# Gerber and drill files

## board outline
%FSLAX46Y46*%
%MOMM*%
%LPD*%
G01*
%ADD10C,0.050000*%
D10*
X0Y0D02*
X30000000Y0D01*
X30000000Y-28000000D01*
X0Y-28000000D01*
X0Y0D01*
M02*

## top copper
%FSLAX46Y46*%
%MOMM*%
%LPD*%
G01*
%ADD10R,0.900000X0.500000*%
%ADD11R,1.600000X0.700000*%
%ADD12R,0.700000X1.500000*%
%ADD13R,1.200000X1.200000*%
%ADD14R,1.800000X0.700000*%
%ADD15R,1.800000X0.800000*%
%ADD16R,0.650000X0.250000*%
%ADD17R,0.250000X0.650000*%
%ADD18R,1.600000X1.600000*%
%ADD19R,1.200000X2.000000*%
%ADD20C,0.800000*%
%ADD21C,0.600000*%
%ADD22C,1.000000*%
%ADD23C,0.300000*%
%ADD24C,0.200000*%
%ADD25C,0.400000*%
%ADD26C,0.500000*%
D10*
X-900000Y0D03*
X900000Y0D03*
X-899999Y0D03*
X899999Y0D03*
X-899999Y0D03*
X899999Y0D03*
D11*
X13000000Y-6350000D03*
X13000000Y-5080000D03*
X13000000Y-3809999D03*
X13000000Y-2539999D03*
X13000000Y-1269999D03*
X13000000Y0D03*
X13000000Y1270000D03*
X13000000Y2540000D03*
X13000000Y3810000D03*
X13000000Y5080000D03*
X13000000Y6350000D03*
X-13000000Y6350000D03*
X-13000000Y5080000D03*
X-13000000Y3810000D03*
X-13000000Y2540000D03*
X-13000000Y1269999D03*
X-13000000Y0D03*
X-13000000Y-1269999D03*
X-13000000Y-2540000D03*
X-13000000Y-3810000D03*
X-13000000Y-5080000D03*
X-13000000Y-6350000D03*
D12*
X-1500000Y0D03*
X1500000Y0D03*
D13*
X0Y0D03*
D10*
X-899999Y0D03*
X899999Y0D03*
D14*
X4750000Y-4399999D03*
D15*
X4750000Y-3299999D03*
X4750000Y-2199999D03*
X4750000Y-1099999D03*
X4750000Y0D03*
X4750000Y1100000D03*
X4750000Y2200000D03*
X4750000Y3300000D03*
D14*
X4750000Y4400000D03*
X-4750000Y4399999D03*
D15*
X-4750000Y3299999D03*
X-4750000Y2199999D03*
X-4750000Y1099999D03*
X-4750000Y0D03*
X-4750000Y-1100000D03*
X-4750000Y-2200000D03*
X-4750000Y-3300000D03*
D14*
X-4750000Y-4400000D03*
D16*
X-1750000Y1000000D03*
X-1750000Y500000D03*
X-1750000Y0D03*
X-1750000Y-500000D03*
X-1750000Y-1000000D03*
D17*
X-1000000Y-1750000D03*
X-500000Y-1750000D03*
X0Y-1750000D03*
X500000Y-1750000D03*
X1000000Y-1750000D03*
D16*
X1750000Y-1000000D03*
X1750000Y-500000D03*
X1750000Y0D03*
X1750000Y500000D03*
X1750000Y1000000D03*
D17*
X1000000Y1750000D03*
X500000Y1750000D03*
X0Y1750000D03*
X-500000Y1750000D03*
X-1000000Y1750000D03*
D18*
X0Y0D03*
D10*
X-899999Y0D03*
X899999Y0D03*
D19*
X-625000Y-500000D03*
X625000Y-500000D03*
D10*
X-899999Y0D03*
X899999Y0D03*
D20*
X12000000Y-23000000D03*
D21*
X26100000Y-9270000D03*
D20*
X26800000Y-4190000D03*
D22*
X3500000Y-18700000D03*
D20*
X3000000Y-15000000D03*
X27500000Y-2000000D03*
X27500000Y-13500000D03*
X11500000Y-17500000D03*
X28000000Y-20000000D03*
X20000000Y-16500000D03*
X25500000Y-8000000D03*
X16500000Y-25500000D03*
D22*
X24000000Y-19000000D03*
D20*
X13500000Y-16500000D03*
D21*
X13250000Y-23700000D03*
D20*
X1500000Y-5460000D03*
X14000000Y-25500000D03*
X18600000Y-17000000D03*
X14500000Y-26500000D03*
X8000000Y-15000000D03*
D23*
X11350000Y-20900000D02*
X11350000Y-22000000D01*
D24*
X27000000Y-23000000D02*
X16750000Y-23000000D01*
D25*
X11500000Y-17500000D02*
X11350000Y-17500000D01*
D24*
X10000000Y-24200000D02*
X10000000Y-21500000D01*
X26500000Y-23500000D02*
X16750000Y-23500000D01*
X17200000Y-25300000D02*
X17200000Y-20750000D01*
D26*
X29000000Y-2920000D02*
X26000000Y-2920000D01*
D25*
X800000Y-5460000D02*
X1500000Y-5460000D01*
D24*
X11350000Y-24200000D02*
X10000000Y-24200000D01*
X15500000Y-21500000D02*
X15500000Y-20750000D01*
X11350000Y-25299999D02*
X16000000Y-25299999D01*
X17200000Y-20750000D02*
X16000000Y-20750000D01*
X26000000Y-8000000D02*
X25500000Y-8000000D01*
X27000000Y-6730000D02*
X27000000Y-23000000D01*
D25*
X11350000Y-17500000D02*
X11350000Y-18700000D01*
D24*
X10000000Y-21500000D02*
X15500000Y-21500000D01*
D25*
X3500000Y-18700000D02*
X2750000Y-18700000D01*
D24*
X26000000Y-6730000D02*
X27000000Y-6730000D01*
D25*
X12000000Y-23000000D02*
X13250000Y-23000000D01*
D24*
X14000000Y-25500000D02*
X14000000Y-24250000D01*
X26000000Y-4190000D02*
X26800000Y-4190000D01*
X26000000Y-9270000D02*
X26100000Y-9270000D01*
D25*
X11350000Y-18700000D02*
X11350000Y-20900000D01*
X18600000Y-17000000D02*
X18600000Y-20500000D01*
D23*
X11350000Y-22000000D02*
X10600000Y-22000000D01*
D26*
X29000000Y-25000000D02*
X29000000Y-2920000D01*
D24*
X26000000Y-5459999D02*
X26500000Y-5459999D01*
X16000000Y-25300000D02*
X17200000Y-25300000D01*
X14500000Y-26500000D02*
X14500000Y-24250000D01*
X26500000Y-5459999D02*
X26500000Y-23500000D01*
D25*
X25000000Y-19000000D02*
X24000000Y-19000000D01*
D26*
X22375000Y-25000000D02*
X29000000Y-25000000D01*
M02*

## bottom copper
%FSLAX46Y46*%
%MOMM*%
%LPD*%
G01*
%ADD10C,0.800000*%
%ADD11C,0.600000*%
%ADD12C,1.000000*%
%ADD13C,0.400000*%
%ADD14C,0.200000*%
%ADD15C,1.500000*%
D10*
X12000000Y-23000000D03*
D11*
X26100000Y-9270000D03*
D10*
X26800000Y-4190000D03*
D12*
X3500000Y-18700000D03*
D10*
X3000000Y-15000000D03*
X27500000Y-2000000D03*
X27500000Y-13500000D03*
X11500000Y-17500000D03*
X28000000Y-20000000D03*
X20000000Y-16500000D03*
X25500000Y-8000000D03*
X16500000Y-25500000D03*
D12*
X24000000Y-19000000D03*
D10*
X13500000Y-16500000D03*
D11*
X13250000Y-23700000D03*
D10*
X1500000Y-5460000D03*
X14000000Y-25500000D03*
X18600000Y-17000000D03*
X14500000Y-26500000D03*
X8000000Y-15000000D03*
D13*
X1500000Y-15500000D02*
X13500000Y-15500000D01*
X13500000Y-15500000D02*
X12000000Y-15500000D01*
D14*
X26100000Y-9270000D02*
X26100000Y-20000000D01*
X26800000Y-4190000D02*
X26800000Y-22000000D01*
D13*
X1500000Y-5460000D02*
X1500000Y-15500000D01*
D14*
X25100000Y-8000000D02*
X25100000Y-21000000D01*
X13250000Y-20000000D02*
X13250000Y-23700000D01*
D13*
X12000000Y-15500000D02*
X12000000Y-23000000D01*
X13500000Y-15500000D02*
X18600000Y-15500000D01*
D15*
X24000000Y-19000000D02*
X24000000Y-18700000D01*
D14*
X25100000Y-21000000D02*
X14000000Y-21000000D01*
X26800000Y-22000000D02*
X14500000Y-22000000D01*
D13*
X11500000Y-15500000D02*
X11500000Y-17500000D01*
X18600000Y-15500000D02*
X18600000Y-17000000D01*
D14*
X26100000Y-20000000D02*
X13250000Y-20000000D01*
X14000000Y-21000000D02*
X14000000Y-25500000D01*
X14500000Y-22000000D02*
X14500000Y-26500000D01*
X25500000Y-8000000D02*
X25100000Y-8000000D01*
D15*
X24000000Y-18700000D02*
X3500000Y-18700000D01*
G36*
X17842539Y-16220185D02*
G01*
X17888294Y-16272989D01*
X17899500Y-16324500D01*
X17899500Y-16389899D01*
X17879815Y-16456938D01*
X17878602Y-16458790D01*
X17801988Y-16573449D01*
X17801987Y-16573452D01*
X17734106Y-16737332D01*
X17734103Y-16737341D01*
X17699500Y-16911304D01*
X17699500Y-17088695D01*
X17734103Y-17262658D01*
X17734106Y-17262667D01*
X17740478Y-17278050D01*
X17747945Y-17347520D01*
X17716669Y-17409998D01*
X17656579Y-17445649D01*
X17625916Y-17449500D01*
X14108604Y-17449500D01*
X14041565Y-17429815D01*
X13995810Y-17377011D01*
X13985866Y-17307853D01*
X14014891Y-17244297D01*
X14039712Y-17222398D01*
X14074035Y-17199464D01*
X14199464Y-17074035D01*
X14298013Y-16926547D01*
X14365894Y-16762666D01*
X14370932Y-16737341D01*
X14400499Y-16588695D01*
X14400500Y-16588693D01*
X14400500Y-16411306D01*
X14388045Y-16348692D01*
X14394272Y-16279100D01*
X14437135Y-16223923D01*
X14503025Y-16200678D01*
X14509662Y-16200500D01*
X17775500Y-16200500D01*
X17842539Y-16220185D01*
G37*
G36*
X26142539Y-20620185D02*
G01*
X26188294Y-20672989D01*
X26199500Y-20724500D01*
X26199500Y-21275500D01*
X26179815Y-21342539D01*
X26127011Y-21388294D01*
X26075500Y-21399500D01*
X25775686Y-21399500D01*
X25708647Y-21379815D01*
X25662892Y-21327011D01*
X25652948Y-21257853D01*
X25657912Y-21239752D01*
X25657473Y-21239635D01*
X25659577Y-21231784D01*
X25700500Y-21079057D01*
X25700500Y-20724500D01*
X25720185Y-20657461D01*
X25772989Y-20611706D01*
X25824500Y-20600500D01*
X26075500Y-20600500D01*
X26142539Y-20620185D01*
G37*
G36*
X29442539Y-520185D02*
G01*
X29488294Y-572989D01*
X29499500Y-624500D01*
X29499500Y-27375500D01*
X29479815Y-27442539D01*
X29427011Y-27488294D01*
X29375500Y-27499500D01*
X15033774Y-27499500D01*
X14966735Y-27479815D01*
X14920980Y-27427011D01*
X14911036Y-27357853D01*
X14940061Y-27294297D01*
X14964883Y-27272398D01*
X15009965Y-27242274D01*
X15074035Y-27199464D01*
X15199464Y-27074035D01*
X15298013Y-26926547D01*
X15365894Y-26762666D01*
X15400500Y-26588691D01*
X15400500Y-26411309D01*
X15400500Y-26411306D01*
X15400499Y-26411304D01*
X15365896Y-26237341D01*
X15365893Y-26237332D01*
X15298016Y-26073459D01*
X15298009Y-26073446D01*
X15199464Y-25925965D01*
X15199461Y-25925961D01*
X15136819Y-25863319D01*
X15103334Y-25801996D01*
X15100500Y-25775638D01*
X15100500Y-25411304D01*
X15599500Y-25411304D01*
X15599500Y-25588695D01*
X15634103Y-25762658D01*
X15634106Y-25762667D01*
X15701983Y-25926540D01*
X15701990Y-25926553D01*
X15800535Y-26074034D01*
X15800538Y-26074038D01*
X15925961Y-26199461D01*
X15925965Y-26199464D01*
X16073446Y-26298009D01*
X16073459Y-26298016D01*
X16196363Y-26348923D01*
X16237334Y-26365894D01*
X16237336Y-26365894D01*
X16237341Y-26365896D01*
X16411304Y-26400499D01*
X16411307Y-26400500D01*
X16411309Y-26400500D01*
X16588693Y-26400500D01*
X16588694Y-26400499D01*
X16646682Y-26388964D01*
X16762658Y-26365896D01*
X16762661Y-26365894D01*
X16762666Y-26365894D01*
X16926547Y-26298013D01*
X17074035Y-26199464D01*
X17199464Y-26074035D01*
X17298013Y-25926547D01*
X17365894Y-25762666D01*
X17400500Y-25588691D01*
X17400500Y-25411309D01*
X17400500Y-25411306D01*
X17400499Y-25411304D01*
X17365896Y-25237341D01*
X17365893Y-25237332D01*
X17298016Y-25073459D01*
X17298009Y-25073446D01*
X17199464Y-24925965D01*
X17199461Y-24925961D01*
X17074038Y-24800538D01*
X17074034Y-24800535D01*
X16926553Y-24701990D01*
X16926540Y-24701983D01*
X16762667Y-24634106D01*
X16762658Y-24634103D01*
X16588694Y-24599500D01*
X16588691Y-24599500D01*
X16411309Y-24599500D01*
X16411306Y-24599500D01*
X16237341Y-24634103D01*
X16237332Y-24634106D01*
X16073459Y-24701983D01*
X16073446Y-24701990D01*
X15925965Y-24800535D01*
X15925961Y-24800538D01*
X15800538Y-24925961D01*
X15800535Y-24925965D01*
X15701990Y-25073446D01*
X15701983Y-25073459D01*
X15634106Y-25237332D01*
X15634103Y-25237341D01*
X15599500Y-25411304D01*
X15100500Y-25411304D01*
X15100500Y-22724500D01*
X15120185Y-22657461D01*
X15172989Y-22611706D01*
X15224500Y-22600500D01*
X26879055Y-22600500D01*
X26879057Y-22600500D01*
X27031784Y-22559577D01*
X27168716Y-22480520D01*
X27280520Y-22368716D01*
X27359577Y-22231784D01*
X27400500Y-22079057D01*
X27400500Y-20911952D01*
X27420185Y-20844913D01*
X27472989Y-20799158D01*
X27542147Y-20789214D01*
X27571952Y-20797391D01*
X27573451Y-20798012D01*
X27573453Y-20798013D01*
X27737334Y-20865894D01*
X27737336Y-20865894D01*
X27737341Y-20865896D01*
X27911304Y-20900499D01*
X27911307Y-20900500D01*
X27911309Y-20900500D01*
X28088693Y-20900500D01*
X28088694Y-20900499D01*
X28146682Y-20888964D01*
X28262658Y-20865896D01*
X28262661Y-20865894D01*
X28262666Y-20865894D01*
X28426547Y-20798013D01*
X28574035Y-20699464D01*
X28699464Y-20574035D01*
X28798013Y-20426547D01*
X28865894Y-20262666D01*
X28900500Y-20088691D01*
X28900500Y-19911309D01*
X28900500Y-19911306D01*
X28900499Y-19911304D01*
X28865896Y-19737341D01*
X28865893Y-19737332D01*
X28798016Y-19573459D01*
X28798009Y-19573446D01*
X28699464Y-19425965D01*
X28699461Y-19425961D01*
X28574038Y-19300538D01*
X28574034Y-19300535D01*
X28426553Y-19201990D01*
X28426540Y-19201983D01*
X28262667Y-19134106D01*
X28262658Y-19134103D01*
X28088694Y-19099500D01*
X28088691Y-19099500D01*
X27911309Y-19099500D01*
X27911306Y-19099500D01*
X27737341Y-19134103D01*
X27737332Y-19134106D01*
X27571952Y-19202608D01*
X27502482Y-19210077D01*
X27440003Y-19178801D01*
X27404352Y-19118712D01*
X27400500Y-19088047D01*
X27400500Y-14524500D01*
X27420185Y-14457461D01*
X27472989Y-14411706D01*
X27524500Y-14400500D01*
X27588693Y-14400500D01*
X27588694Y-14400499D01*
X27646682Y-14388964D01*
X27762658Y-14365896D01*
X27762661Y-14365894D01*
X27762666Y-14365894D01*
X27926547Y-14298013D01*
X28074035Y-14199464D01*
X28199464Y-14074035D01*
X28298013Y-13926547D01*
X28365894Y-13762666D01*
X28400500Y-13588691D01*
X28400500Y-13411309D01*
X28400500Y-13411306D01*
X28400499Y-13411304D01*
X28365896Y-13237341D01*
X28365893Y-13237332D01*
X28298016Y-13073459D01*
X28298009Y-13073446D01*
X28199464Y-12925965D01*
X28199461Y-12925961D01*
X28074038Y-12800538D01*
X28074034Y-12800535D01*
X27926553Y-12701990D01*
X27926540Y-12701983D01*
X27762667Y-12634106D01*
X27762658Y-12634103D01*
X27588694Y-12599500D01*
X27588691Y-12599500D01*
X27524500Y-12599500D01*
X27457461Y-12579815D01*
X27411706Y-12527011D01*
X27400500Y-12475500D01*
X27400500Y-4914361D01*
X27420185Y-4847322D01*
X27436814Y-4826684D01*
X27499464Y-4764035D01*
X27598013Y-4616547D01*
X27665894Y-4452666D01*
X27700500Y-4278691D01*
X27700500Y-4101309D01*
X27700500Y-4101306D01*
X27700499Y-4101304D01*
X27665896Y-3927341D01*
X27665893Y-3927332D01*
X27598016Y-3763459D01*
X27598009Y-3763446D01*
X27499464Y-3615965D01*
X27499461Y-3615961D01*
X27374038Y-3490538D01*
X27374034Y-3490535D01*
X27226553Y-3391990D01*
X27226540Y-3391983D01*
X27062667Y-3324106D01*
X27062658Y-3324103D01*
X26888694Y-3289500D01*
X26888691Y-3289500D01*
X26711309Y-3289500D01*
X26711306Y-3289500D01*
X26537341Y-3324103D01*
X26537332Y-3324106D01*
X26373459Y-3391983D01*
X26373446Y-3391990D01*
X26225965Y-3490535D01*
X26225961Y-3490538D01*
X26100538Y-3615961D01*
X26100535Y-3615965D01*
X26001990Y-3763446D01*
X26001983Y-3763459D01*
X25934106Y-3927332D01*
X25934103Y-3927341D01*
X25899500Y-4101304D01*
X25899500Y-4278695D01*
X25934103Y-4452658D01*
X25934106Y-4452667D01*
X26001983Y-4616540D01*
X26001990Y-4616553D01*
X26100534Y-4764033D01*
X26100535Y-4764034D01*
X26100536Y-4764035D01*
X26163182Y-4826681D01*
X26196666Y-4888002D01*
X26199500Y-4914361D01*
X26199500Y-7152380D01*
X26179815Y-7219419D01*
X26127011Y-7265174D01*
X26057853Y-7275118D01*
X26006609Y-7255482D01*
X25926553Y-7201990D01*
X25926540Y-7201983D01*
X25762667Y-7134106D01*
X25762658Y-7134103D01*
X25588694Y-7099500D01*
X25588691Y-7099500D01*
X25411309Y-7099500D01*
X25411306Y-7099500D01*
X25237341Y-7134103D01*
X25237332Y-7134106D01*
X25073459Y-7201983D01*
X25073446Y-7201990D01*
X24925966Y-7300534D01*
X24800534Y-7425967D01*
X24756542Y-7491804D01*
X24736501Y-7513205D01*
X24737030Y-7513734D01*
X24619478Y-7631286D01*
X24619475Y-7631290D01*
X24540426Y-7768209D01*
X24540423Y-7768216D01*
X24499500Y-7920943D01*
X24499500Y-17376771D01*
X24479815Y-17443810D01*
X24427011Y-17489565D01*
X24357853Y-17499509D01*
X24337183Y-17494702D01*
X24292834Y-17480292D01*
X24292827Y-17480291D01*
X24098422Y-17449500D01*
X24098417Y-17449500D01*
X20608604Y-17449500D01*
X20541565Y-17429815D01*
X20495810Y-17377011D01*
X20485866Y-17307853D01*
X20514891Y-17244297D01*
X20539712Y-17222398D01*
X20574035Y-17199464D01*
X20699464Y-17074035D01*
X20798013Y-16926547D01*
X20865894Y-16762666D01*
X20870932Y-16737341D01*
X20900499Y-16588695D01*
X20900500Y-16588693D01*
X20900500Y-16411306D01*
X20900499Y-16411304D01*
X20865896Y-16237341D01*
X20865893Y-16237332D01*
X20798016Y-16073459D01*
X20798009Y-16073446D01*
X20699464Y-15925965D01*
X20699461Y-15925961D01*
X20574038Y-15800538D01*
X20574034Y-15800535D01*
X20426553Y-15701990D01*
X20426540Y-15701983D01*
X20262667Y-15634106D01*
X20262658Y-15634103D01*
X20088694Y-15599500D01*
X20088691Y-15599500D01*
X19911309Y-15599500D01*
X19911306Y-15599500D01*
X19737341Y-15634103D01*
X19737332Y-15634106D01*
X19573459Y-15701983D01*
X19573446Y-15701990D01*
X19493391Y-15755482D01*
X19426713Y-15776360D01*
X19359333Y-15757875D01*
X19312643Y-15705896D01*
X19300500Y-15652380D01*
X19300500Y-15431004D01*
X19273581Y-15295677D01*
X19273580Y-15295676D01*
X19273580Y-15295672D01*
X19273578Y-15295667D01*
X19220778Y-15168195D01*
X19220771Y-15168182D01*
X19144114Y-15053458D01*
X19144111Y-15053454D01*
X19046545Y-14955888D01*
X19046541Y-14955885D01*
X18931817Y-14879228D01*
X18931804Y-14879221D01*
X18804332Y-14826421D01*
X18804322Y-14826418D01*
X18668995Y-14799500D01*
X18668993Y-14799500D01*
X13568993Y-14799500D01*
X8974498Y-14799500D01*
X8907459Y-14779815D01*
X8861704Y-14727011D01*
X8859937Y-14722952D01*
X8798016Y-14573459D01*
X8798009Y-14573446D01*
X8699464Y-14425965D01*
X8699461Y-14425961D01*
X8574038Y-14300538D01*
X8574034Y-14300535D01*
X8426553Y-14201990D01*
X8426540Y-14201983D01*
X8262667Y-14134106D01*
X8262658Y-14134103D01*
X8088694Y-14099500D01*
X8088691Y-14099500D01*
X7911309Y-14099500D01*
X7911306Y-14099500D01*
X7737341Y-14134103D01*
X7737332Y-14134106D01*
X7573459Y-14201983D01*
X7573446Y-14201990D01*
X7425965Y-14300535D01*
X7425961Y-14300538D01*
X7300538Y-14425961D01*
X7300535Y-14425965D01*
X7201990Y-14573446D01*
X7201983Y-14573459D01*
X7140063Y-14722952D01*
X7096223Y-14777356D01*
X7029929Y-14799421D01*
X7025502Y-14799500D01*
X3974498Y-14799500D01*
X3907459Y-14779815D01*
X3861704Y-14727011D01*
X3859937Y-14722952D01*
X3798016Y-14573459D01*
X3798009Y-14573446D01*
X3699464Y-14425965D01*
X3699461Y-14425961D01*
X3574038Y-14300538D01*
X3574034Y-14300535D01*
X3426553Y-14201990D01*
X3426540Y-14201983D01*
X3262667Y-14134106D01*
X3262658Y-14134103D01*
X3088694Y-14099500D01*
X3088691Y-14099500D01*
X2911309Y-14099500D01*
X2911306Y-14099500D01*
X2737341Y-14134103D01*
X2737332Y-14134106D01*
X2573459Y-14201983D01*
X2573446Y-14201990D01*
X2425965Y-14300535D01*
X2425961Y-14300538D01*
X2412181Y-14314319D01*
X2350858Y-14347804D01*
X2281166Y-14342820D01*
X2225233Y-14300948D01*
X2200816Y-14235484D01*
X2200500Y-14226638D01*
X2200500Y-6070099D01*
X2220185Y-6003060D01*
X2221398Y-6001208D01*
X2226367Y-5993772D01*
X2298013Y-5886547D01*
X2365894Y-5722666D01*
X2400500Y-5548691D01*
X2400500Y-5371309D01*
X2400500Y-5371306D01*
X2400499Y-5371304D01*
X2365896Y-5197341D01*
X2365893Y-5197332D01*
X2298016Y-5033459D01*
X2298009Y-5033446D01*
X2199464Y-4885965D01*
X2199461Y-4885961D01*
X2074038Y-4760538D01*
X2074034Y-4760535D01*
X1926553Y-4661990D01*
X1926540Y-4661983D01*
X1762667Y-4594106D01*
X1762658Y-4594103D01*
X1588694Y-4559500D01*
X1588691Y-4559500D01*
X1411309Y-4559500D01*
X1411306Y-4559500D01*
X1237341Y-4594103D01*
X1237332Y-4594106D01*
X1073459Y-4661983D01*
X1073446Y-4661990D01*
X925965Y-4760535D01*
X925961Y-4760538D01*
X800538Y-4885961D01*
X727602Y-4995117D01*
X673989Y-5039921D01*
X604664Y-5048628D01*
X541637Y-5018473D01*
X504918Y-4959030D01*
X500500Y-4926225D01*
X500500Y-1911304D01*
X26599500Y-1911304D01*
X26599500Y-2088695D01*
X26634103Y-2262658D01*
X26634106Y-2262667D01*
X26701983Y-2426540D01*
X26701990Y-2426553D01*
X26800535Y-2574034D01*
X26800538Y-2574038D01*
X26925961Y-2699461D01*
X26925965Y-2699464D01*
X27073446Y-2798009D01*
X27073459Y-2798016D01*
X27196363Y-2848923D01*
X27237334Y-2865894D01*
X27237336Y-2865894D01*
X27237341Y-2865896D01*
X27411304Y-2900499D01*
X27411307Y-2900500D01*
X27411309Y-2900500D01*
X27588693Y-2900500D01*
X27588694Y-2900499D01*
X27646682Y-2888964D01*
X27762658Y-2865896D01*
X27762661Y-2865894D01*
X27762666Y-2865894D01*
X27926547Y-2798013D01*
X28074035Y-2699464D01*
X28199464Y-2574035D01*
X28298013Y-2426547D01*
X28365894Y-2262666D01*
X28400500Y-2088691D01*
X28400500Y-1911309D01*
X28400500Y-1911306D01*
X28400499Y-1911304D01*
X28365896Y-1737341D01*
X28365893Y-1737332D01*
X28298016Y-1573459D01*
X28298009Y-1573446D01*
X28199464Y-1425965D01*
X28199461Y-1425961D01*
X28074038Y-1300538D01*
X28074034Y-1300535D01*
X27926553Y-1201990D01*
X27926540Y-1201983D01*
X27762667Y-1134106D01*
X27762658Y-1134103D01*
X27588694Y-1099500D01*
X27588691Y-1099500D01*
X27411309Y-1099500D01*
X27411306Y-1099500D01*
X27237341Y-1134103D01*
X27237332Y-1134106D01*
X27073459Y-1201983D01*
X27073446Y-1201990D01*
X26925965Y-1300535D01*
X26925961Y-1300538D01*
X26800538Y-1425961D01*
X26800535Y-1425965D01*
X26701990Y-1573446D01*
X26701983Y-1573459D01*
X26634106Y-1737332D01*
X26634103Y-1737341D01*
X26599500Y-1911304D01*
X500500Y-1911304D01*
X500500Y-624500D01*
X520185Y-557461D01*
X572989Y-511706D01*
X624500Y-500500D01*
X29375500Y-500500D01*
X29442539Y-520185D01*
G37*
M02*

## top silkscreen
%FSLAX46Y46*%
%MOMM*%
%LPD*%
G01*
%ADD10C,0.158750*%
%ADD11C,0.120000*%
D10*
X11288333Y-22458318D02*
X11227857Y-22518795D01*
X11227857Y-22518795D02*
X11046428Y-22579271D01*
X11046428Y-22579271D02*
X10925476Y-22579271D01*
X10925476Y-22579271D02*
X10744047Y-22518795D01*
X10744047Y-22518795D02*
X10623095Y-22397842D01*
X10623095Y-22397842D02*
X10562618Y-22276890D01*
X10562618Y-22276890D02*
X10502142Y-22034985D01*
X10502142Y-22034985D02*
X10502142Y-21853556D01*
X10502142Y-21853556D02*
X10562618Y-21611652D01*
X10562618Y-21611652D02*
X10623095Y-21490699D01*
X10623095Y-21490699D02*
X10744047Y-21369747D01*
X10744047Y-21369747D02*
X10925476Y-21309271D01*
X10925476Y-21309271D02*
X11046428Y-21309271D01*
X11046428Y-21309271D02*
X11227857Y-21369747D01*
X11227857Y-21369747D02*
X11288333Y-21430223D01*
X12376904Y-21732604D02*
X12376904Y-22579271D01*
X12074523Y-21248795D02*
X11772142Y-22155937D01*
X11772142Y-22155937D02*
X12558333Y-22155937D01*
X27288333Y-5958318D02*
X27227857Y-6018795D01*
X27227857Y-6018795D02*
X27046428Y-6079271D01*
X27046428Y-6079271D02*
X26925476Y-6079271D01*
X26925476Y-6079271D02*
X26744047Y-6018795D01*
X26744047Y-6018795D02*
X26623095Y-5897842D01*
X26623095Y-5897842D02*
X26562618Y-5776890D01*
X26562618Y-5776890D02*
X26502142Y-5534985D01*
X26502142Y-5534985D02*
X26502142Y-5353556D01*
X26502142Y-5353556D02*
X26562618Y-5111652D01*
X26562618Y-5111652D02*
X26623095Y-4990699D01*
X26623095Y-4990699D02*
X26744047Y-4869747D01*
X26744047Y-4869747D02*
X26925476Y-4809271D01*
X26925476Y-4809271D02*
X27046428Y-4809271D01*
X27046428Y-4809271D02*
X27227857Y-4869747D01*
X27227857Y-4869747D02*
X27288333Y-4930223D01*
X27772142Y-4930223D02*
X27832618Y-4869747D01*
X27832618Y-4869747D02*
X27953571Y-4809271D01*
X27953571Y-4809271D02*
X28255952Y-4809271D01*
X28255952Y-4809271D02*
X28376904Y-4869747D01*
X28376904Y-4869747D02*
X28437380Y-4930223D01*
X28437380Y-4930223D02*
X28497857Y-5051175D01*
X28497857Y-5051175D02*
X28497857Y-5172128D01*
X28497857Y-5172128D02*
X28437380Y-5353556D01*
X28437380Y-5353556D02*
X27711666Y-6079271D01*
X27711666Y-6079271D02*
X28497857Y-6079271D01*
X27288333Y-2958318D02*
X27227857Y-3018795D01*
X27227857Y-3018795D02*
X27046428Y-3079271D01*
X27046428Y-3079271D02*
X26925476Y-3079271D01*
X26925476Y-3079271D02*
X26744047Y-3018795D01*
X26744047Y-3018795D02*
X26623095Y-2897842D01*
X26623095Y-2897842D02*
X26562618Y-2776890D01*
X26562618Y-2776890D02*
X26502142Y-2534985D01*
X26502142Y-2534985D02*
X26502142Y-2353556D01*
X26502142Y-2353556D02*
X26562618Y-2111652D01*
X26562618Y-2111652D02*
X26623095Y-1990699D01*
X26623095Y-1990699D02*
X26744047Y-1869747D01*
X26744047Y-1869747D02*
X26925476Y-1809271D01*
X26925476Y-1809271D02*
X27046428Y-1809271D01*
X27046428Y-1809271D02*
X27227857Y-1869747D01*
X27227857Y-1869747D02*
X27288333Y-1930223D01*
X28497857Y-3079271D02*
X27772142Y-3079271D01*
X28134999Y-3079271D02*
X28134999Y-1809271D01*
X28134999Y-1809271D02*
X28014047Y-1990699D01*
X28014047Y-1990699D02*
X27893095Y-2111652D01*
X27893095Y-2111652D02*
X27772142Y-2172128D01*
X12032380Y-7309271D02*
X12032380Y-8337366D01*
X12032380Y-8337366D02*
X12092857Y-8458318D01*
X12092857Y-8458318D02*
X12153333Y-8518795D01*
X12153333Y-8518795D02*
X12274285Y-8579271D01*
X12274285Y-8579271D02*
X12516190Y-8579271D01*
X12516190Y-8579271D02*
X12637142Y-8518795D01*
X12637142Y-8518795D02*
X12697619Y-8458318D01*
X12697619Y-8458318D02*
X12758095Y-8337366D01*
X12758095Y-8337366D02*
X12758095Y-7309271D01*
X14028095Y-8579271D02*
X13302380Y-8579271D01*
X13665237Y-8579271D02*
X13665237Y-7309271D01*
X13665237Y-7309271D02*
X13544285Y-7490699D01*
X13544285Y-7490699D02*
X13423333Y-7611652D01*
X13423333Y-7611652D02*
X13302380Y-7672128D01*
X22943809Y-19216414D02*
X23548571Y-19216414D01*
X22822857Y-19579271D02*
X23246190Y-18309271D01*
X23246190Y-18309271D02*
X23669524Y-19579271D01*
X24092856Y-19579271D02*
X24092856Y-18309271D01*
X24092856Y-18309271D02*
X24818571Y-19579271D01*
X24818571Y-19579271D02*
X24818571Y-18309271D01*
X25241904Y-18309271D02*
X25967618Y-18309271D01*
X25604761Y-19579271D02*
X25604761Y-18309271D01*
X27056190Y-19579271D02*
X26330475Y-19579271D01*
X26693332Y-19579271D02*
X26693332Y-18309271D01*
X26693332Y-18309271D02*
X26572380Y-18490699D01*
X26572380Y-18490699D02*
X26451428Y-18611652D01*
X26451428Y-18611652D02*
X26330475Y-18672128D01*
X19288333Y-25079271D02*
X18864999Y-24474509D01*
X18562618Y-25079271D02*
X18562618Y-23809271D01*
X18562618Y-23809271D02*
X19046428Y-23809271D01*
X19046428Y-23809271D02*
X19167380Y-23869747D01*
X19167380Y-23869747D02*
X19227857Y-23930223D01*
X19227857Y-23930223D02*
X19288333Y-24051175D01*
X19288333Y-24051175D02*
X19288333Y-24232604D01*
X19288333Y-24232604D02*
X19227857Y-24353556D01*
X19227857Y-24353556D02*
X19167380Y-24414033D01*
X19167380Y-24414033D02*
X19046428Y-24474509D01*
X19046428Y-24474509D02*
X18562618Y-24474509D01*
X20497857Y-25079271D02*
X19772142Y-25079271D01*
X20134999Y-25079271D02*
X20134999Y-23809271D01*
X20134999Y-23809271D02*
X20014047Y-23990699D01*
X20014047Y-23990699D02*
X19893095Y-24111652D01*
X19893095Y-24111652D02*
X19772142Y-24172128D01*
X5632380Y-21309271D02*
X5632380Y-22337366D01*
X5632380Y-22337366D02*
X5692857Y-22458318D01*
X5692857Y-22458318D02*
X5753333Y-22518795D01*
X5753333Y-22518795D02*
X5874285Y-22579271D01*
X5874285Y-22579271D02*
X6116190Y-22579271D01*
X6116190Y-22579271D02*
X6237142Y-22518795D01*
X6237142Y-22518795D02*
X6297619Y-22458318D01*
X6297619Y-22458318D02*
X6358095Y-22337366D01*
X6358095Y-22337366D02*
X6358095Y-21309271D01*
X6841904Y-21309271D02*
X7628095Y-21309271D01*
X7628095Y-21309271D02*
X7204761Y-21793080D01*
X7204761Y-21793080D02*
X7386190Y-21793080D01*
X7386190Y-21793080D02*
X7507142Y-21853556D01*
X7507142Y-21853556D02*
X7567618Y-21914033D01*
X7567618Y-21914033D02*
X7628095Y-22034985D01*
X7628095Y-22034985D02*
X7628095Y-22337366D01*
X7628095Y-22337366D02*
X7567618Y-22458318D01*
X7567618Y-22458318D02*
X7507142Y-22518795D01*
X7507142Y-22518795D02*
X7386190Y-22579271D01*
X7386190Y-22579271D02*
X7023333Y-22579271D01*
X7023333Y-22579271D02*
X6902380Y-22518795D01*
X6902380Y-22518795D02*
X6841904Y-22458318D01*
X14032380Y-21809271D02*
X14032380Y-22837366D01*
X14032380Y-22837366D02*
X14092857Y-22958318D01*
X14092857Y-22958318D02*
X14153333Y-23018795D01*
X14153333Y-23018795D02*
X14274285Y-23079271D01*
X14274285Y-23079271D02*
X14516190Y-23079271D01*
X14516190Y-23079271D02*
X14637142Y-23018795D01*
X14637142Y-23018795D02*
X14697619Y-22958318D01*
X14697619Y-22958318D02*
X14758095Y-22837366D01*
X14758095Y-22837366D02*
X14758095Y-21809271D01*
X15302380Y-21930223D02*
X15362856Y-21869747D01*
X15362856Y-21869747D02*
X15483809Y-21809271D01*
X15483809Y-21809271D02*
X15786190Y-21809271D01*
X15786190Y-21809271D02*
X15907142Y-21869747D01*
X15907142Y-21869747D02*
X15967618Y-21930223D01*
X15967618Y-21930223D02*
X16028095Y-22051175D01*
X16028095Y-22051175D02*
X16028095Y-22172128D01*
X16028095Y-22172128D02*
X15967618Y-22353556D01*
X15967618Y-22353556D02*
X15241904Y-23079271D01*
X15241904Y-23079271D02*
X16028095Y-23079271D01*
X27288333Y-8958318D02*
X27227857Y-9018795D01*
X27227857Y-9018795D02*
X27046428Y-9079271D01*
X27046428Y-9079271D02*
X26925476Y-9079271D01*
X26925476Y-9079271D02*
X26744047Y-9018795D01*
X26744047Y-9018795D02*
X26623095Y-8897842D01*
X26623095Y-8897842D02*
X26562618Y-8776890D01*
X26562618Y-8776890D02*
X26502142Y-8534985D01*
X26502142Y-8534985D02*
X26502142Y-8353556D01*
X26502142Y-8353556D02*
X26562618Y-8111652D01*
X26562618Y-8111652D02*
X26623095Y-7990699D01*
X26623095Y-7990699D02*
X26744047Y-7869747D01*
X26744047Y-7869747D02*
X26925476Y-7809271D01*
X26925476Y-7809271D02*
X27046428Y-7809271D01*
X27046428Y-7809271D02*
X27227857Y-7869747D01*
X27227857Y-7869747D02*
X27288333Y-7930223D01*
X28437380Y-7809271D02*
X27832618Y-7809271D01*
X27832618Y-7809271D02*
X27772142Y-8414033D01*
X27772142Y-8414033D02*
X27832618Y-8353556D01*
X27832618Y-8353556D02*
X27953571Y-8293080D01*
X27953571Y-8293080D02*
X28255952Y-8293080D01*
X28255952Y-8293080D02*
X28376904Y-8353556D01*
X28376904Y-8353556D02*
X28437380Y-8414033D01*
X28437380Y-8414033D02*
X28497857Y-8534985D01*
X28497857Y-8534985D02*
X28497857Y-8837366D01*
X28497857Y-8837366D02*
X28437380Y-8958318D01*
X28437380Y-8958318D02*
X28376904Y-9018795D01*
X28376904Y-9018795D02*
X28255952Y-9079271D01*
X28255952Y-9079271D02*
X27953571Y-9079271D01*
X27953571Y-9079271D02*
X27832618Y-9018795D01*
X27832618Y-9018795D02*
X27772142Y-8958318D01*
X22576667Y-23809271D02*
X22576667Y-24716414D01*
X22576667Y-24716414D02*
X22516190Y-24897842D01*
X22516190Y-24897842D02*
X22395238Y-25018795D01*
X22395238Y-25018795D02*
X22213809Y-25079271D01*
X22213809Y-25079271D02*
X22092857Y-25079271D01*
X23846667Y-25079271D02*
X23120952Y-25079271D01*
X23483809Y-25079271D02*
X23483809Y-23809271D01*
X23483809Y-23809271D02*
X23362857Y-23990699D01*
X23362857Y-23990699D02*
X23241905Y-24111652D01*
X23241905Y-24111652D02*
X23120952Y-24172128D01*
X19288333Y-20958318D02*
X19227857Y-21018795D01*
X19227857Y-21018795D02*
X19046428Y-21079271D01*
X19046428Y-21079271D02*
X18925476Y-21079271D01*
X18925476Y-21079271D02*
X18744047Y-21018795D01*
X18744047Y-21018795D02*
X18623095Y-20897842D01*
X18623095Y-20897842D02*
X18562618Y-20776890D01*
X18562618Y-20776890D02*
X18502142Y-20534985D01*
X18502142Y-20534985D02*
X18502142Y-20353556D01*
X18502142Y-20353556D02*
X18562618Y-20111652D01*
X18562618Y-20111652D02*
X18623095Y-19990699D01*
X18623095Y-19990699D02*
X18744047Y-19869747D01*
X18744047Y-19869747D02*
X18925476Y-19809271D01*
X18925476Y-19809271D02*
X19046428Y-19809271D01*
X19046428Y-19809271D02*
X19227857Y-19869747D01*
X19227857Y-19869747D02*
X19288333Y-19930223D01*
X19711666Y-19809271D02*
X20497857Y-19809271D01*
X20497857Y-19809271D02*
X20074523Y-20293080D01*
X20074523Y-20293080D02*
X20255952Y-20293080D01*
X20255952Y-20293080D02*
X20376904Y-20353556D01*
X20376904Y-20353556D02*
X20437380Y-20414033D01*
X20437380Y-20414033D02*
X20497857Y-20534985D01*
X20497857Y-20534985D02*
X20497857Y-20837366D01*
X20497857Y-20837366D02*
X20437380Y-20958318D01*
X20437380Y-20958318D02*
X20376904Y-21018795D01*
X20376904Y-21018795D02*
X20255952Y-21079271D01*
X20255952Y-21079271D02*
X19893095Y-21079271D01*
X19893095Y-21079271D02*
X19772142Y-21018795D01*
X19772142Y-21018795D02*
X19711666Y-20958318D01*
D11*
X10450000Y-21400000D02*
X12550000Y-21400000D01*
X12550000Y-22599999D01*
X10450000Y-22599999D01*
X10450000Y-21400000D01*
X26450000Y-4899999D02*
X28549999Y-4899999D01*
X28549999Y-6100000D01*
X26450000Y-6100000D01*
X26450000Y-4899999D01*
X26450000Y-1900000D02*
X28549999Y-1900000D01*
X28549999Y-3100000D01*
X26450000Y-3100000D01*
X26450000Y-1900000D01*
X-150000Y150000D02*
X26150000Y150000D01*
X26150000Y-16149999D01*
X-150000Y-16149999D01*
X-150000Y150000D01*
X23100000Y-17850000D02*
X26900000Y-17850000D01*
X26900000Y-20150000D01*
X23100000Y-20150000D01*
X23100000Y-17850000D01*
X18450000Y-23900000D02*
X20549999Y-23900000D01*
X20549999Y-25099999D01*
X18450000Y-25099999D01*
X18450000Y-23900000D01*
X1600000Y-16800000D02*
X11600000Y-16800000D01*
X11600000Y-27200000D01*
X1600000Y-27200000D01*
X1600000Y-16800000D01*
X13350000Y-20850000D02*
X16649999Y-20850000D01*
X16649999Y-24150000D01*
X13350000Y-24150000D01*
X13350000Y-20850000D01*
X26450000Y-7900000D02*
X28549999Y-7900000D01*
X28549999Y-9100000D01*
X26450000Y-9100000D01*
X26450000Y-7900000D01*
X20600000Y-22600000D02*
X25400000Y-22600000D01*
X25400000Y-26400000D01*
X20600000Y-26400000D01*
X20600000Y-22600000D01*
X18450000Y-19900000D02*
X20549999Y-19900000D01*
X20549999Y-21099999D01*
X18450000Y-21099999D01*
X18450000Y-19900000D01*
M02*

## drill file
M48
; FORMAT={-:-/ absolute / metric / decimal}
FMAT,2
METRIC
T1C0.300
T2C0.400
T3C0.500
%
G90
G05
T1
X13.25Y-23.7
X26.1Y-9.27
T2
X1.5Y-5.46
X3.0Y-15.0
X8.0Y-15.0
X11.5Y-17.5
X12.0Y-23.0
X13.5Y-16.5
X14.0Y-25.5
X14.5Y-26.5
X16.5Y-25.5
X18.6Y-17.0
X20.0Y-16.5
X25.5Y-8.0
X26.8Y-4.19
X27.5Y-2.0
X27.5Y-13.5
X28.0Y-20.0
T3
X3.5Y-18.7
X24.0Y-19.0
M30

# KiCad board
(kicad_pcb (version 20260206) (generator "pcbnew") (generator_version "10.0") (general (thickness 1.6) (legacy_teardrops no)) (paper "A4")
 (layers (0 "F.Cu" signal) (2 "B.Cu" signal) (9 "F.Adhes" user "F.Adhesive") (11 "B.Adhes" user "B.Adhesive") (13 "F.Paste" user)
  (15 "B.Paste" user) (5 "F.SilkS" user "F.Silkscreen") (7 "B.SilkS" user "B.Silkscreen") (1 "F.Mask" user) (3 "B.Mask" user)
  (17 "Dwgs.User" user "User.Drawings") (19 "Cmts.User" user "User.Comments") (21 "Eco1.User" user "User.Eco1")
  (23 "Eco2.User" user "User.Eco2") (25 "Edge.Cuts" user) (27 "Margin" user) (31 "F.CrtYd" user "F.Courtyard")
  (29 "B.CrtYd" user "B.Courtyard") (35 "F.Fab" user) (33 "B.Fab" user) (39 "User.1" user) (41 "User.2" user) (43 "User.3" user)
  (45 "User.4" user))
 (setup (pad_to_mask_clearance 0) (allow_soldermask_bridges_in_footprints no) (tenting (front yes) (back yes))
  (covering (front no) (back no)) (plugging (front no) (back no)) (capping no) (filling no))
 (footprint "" (layer "F.Cu") (at 11.5 22)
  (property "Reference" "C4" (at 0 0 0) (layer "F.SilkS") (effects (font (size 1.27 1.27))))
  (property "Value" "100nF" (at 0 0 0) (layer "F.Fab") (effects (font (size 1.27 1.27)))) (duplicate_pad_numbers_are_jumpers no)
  (fp_rect (start -1.05 -0.6) (end 1.05 0.599999) (stroke (width 0.12) (type default)) (fill no) (layer "F.SilkS"))
  (pad "1" smd rect (at -12.4 -22) (size 0.9 0.5) (layers "F.Cu" "F.Mask" "F.Paste") (thermal_bridge_angle 45))
  (pad "2" smd rect (at -10.6 -22) (size 0.9 0.5) (layers "F.Cu" "F.Mask" "F.Paste") (thermal_bridge_angle 45)))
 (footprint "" (layer "F.Cu") (at 27.5 5.5)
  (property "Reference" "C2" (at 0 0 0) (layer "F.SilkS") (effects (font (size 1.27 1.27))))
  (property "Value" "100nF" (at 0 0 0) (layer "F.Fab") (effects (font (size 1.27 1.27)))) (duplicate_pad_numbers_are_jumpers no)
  (fp_rect (start -1.05 -0.600001) (end 1.049999 0.6) (stroke (width 0.12) (type default)) (fill no) (layer "F.SilkS"))
  (pad "1" smd rect (at -28.399999 -5.5) (size 0.9 0.5) (layers "F.Cu" "F.Mask" "F.Paste") (thermal_bridge_angle 45))
  (pad "2" smd rect (at -26.600001 -5.5) (size 0.9 0.5) (layers "F.Cu" "F.Mask" "F.Paste") (thermal_bridge_angle 45)))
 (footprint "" (layer "F.Cu") (at 27.5 2.5)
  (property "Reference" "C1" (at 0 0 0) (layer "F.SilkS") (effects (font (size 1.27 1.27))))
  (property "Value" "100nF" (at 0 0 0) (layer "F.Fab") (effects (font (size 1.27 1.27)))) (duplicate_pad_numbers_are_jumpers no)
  (fp_rect (start -1.05 -0.6) (end 1.049999 0.6) (stroke (width 0.12) (type default)) (fill no) (layer "F.SilkS"))
  (pad "1" smd rect (at -28.399999 -2.5) (size 0.9 0.5) (layers "F.Cu" "F.Mask" "F.Paste") (thermal_bridge_angle 45))
  (pad "2" smd rect (at -26.600001 -2.5) (size 0.9 0.5) (layers "F.Cu" "F.Mask" "F.Paste") (thermal_bridge_angle 45)))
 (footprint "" (layer "F.Cu") (at 13 8)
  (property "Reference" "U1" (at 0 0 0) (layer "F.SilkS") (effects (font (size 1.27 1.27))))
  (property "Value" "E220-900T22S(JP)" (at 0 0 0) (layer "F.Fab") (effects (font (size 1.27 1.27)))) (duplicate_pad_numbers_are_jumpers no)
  (fp_rect (start -13.15 -8.15) (end 13.15 8.149999) (stroke (width 0.12) (type default)) (fill no) (layer "F.SilkS"))
  (pad "1" smd rect (at 0 -1.65) (size 1.6 0.7) (layers "F.Cu" "F.Mask" "F.Paste") (thermal_bridge_angle 45))
  (pad "2" smd rect (at 0 -2.92) (size 1.6 0.7) (layers "F.Cu" "F.Mask" "F.Paste") (thermal_bridge_angle 45))
  (pad "3" smd rect (at 0 -4.190001) (size 1.6 0.7) (layers "F.Cu" "F.Mask" "F.Paste") (thermal_bridge_angle 45))
  (pad "4" smd rect (at 0 -5.460001) (size 1.6 0.7) (layers "F.Cu" "F.Mask" "F.Paste") (thermal_bridge_angle 45))
  (pad "5" smd rect (at 0 -6.730001) (size 1.6 0.7) (layers "F.Cu" "F.Mask" "F.Paste") (thermal_bridge_angle 45))
  (pad "6" smd rect (at 0 -8) (size 1.6 0.7) (layers "F.Cu" "F.Mask" "F.Paste") (thermal_bridge_angle 45))
  (pad "7" smd rect (at 0 -9.27) (size 1.6 0.7) (layers "F.Cu" "F.Mask" "F.Paste") (thermal_bridge_angle 45))
  (pad "8" smd rect (at 0 -10.54) (size 1.6 0.7) (layers "F.Cu" "F.Mask" "F.Paste") (thermal_bridge_angle 45))
  (pad "9" smd rect (at 0 -11.81) (size 1.6 0.7) (layers "F.Cu" "F.Mask" "F.Paste") (thermal_bridge_angle 45))
  (pad "10" smd rect (at 0 -13.08) (size 1.6 0.7) (layers "F.Cu" "F.Mask" "F.Paste") (thermal_bridge_angle 45))
  (pad "11" smd rect (at 0 -14.35) (size 1.6 0.7) (layers "F.Cu" "F.Mask" "F.Paste") (thermal_bridge_angle 45))
  (pad "12" smd rect (at -26 -14.35) (size 1.6 0.7) (layers "F.Cu" "F.Mask" "F.Paste") (thermal_bridge_angle 45))
  (pad "13" smd rect (at -26 -13.08) (size 1.6 0.7) (layers "F.Cu" "F.Mask" "F.Paste") (thermal_bridge_angle 45))
  (pad "14" smd rect (at -26 -11.81) (size 1.6 0.7) (layers "F.Cu" "F.Mask" "F.Paste") (thermal_bridge_angle 45))
  (pad "15" smd rect (at -26 -10.54) (size 1.6 0.7) (layers "F.Cu" "F.Mask" "F.Paste") (thermal_bridge_angle 45))
  (pad "16" smd rect (at -26 -9.269999) (size 1.6 0.7) (layers "F.Cu" "F.Mask" "F.Paste") (thermal_bridge_angle 45))
  (pad "17" smd rect (at -26 -8) (size 1.6 0.7) (layers "F.Cu" "F.Mask" "F.Paste") (thermal_bridge_angle 45))
  (pad "18" smd rect (at -26 -6.730001) (size 1.6 0.7) (layers "F.Cu" "F.Mask" "F.Paste") (thermal_bridge_angle 45))
  (pad "19" smd rect (at -26 -5.46) (size 1.6 0.7) (layers "F.Cu" "F.Mask" "F.Paste") (thermal_bridge_angle 45))
  (pad "20" smd rect (at -26 -4.19) (size 1.6 0.7) (layers "F.Cu" "F.Mask" "F.Paste") (thermal_bridge_angle 45))
  (pad "21" smd rect (at -26 -2.92) (size 1.6 0.7) (layers "F.Cu" "F.Mask" "F.Paste") (thermal_bridge_angle 45))
  (pad "22" smd rect (at -26 -1.65) (size 1.6 0.7) (layers "F.Cu" "F.Mask" "F.Paste") (thermal_bridge_angle 45)))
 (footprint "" (layer "F.Cu") (at 25 19)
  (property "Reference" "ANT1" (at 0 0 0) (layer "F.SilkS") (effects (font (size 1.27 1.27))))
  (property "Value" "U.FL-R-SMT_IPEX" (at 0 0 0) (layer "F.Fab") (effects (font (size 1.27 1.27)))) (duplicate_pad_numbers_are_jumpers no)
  (fp_rect (start -1.9 -1.15) (end 1.9 1.15) (stroke (width 0.12) (type default)) (fill no) (layer "F.SilkS"))
  (pad "G1" smd rect (at -26.5 -19) (size 0.7 1.5) (layers "F.Cu" "F.Mask" "F.Paste") (thermal_bridge_angle 45))
  (pad "G2" smd rect (at -23.5 -19) (size 0.7 1.5) (layers "F.Cu" "F.Mask" "F.Paste") (thermal_bridge_angle 45))
  (pad "S" smd rect (at -25 -19) (size 1.2 1.2) (layers "F.Cu" "F.Mask" "F.Paste") (thermal_bridge_angle 45)))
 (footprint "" (layer "F.Cu") (at 19.5 24.5)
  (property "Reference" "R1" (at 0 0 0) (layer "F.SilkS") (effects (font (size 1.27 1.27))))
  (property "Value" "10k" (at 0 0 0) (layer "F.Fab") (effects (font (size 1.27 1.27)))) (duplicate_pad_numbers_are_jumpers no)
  (fp_rect (start -1.05 -0.6) (end 1.049999 0.599999) (stroke (width 0.12) (type default)) (fill no) (layer "F.SilkS"))
  (pad "1" smd rect (at -20.399999 -24.5) (size 0.9 0.5) (layers "F.Cu" "F.Mask" "F.Paste") (thermal_bridge_angle 45))
  (pad "2" smd rect (at -18.600001 -24.5) (size 0.9 0.5) (layers "F.Cu" "F.Mask" "F.Paste") (thermal_bridge_angle 45)))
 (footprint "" (layer "F.Cu") (at 6.6 22)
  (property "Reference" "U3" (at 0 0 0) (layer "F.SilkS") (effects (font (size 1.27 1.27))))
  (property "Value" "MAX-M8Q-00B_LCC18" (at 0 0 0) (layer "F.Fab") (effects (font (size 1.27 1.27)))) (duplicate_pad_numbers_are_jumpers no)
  (fp_rect (start -5 -5.2) (end 5 5.2) (stroke (width 0.12) (type default)) (fill no) (layer "F.SilkS"))
  (pad "1" smd rect (at -1.85 -17.600001) (size 1.8 0.7) (layers "F.Cu" "F.Mask" "F.Paste") (thermal_bridge_angle 45))
  (pad "2" smd rect (at -1.85 -18.700001) (size 1.8 0.8) (layers "F.Cu" "F.Mask" "F.Paste") (thermal_bridge_angle 45))
  (pad "3" smd rect (at -1.85 -19.800001) (size 1.8 0.8) (layers "F.Cu" "F.Mask" "F.Paste") (thermal_bridge_angle 45))
  (pad "4" smd rect (at -1.85 -20.900001) (size 1.8 0.8) (layers "F.Cu" "F.Mask" "F.Paste") (thermal_bridge_angle 45))
  (pad "5" smd rect (at -1.85 -22) (size 1.8 0.8) (layers "F.Cu" "F.Mask" "F.Paste") (thermal_bridge_angle 45))
  (pad "6" smd rect (at -1.85 -23.1) (size 1.8 0.8) (layers "F.Cu" "F.Mask" "F.Paste") (thermal_bridge_angle 45))
  (pad "7" smd rect (at -1.85 -24.2) (size 1.8 0.8) (layers "F.Cu" "F.Mask" "F.Paste") (thermal_bridge_angle 45))
  (pad "8" smd rect (at -1.85 -25.3) (size 1.8 0.8) (layers "F.Cu" "F.Mask" "F.Paste") (thermal_bridge_angle 45))
  (pad "9" smd rect (at -1.85 -26.4) (size 1.8 0.7) (layers "F.Cu" "F.Mask" "F.Paste") (thermal_bridge_angle 45))
  (pad "10" smd rect (at -11.35 -26.399999) (size 1.8 0.7) (layers "F.Cu" "F.Mask" "F.Paste") (thermal_bridge_angle 45))
  (pad "11" smd rect (at -11.35 -25.299999) (size 1.8 0.8) (layers "F.Cu" "F.Mask" "F.Paste") (thermal_bridge_angle 45))
  (pad "12" smd rect (at -11.35 -24.199999) (size 1.8 0.8) (layers "F.Cu" "F.Mask" "F.Paste") (thermal_bridge_angle 45))
  (pad "13" smd rect (at -11.35 -23.099999) (size 1.8 0.8) (layers "F.Cu" "F.Mask" "F.Paste") (thermal_bridge_angle 45))
  (pad "14" smd rect (at -11.35 -22) (size 1.8 0.8) (layers "F.Cu" "F.Mask" "F.Paste") (thermal_bridge_angle 45))
  (pad "15" smd rect (at -11.35 -20.9) (size 1.8 0.8) (layers "F.Cu" "F.Mask" "F.Paste") (thermal_bridge_angle 45))
  (pad "16" smd rect (at -11.35 -19.8) (size 1.8 0.8) (layers "F.Cu" "F.Mask" "F.Paste") (thermal_bridge_angle 45))
  (pad "17" smd rect (at -11.35 -18.7) (size 1.8 0.8) (layers "F.Cu" "F.Mask" "F.Paste") (thermal_bridge_angle 45))
  (pad "18" smd rect (at -11.35 -17.6) (size 1.8 0.7) (layers "F.Cu" "F.Mask" "F.Paste") (thermal_bridge_angle 45)))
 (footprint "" (layer "F.Cu") (at 15 22.5)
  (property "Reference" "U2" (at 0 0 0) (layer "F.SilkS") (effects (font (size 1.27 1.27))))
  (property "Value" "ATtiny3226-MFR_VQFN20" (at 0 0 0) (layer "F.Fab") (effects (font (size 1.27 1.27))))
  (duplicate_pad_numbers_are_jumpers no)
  (fp_rect (start -1.65 -1.65) (end 1.649999 1.65) (stroke (width 0.12) (type default)) (fill no) (layer "F.SilkS"))
  (pad "1" smd rect (at -16.75 -23.5) (size 0.65 0.25) (layers "F.Cu" "F.Mask" "F.Paste") (thermal_bridge_angle 45))
  (pad "2" smd rect (at -16.75 -23) (size 0.65 0.25) (layers "F.Cu" "F.Mask" "F.Paste") (thermal_bridge_angle 45))
  (pad "3" smd rect (at -16.75 -22.5) (size 0.65 0.25) (layers "F.Cu" "F.Mask" "F.Paste") (thermal_bridge_angle 45))
  (pad "4" smd rect (at -16.75 -22) (size 0.65 0.25) (layers "F.Cu" "F.Mask" "F.Paste") (thermal_bridge_angle 45))
  (pad "5" smd rect (at -16.75 -21.5) (size 0.65 0.25) (layers "F.Cu" "F.Mask" "F.Paste") (thermal_bridge_angle 45))
  (pad "6" smd rect (at -16 -20.75) (size 0.25 0.65) (layers "F.Cu" "F.Mask" "F.Paste") (thermal_bridge_angle 45))
  (pad "7" smd rect (at -15.5 -20.75) (size 0.25 0.65) (layers "F.Cu" "F.Mask" "F.Paste") (thermal_bridge_angle 45))
  (pad "8" smd rect (at -15 -20.75) (size 0.25 0.65) (layers "F.Cu" "F.Mask" "F.Paste") (thermal_bridge_angle 45))
  (pad "9" smd rect (at -14.5 -20.75) (size 0.25 0.65) (layers "F.Cu" "F.Mask" "F.Paste") (thermal_bridge_angle 45))
  (pad "10" smd rect (at -14 -20.75) (size 0.25 0.65) (layers "F.Cu" "F.Mask" "F.Paste") (thermal_bridge_angle 45))
  (pad "11" smd rect (at -13.25 -21.5) (size 0.65 0.25) (layers "F.Cu" "F.Mask" "F.Paste") (thermal_bridge_angle 45))
  (pad "12" smd rect (at -13.25 -22) (size 0.65 0.25) (layers "F.Cu" "F.Mask" "F.Paste") (thermal_bridge_angle 45))
  (pad "13" smd rect (at -13.25 -22.5) (size 0.65 0.25) (layers "F.Cu" "F.Mask" "F.Paste") (thermal_bridge_angle 45))
  (pad "14" smd rect (at -13.25 -23) (size 0.65 0.25) (layers "F.Cu" "F.Mask" "F.Paste") (thermal_bridge_angle 45))
  (pad "15" smd rect (at -13.25 -23.5) (size 0.65 0.25) (layers "F.Cu" "F.Mask" "F.Paste") (thermal_bridge_angle 45))
  (pad "16" smd rect (at -14 -24.25) (size 0.25 0.65) (layers "F.Cu" "F.Mask" "F.Paste") (thermal_bridge_angle 45))
  (pad "17" smd rect (at -14.5 -24.25) (size 0.25 0.65) (layers "F.Cu" "F.Mask" "F.Paste") (thermal_bridge_angle 45))
  (pad "18" smd rect (at -15 -24.25) (size 0.25 0.65) (layers "F.Cu" "F.Mask" "F.Paste") (thermal_bridge_angle 45))
  (pad "19" smd rect (at -15.5 -24.25) (size 0.25 0.65) (layers "F.Cu" "F.Mask" "F.Paste") (thermal_bridge_angle 45))
  (pad "20" smd rect (at -16 -24.25) (size 0.25 0.65) (layers "F.Cu" "F.Mask" "F.Paste") (thermal_bridge_angle 45))
  (pad "EP" smd rect (at -15 -22.5) (size 1.6 1.6) (layers "F.Cu" "F.Mask" "F.Paste") (thermal_bridge_angle 45)))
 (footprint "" (layer "F.Cu") (at 27.5 8.5)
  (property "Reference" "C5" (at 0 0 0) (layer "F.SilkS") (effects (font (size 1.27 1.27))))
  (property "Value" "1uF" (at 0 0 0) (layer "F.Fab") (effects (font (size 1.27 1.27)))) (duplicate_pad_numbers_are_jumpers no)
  (fp_rect (start -1.05 -0.6) (end 1.049999 0.6) (stroke (width 0.12) (type default)) (fill no) (layer "F.SilkS"))
  (pad "1" smd rect (at -28.399999 -8.5) (size 0.9 0.5) (layers "F.Cu" "F.Mask" "F.Paste") (thermal_bridge_angle 45))
  (pad "2" smd rect (at -26.600001 -8.5) (size 0.9 0.5) (layers "F.Cu" "F.Mask" "F.Paste") (thermal_bridge_angle 45)))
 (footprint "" (layer "F.Cu") (at 23 24.5)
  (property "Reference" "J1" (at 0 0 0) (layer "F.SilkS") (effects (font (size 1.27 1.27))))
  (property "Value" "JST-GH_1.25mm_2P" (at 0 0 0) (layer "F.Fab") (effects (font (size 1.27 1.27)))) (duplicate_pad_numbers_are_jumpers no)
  (fp_rect (start -2.4 -1.9) (end 2.4 1.9) (stroke (width 0.12) (type default)) (fill no) (layer "F.SilkS"))
  (pad "1" smd rect (at -23.625 -24) (size 1.2 2) (layers "F.Cu" "F.Mask" "F.Paste") (thermal_bridge_angle 45))
  (pad "2" smd rect (at -22.375 -24) (size 1.2 2) (layers "F.Cu" "F.Mask" "F.Paste") (thermal_bridge_angle 45)))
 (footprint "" (layer "F.Cu") (at 19.5 20.5)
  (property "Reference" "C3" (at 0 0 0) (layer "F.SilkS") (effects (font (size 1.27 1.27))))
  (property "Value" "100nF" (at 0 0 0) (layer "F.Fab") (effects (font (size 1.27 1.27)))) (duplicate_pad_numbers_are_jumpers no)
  (fp_rect (start -1.05 -0.6) (end 1.049999 0.599999) (stroke (width 0.12) (type default)) (fill no) (layer "F.SilkS"))
  (pad "1" smd rect (at -20.399999 -20.5) (size 0.9 0.5) (layers "F.Cu" "F.Mask" "F.Paste") (thermal_bridge_angle 45))
  (pad "2" smd rect (at -18.600001 -20.5) (size 0.9 0.5) (layers "F.Cu" "F.Mask" "F.Paste") (thermal_bridge_angle 45)))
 (gr_rect (start 0 0) (end 30 28) (stroke (width 0.05) (type default)) (fill no) (layer "Edge.Cuts"))
 (segment (start 11.35 20.9) (end 11.35 22) (width 0.3) (layer "F.Cu") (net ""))
 (segment (start 27 23) (end 16.75 23) (width 0.2) (layer "F.Cu") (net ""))
 (segment (start 11.5 17.5) (end 11.35 17.5) (width 0.4) (layer "F.Cu") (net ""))
 (segment (start 10 24.2) (end 10 21.5) (width 0.2) (layer "F.Cu") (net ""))
 (segment (start 26.5 23.5) (end 16.75 23.5) (width 0.2) (layer "F.Cu") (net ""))
 (segment (start 17.2 25.3) (end 17.2 20.75) (width 0.2) (layer "F.Cu") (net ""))
 (segment (start 29 2.92) (end 26 2.92) (width 0.5) (layer "F.Cu") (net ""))
 (segment (start 0.8 5.46) (end 1.5 5.46) (width 0.4) (layer "F.Cu") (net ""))
 (segment (start 11.35 24.2) (end 10 24.2) (width 0.2) (layer "F.Cu") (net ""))
 (segment (start 15.5 21.5) (end 15.5 20.75) (width 0.2) (layer "F.Cu") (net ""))
 (segment (start 11.35 25.299999) (end 16 25.299999) (width 0.2) (layer "F.Cu") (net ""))
 (segment (start 17.2 20.75) (end 16 20.75) (width 0.2) (layer "F.Cu") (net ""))
 (segment (start 26 8) (end 25.5 8) (width 0.2) (layer "F.Cu") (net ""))
 (segment (start 27 6.73) (end 27 23) (width 0.2) (layer "F.Cu") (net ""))
 (segment (start 11.35 17.5) (end 11.35 18.7) (width 0.4) (layer "F.Cu") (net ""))
 (segment (start 10 21.5) (end 15.5 21.5) (width 0.2) (layer "F.Cu") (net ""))
 (segment (start 3.5 18.7) (end 2.75 18.7) (width 0.4) (layer "F.Cu") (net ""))
 (segment (start 26 6.73) (end 27 6.73) (width 0.2) (layer "F.Cu") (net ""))
 (segment (start 12 23) (end 13.25 23) (width 0.4) (layer "F.Cu") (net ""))
 (segment (start 14 25.5) (end 14 24.25) (width 0.2) (layer "F.Cu") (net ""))
 (segment (start 26 4.19) (end 26.8 4.19) (width 0.2) (layer "F.Cu") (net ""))
 (segment (start 26 9.27) (end 26.1 9.27) (width 0.2) (layer "F.Cu") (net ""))
 (segment (start 11.35 18.7) (end 11.35 20.9) (width 0.4) (layer "F.Cu") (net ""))
 (segment (start 18.6 17) (end 18.6 20.5) (width 0.4) (layer "F.Cu") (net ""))
 (segment (start 11.35 22) (end 10.6 22) (width 0.3) (layer "F.Cu") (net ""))
 (segment (start 29 25) (end 29 2.92) (width 0.5) (layer "F.Cu") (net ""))
 (segment (start 26 5.459999) (end 26.5 5.459999) (width 0.2) (layer "F.Cu") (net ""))
 (segment (start 16 25.3) (end 17.2 25.3) (width 0.2) (layer "F.Cu") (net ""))
 (segment (start 14.5 26.5) (end 14.5 24.25) (width 0.2) (layer "F.Cu") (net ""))
 (segment (start 26.5 5.459999) (end 26.5 23.5) (width 0.2) (layer "F.Cu") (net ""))
 (segment (start 25 19) (end 24 19) (width 0.4) (layer "F.Cu") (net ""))
 (segment (start 22.375 25) (end 29 25) (width 0.5) (layer "F.Cu") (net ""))
 (via (at 12 23) (size 0.8) (drill 0.4) (layers "F.Cu" "B.Cu") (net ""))
 (via (at 26.1 9.27) (size 0.6) (drill 0.3) (layers "F.Cu" "B.Cu") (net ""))
 (via (at 26.8 4.19) (size 0.8) (drill 0.4) (layers "F.Cu" "B.Cu") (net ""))
 (via (at 3.5 18.7) (size 1) (drill 0.5) (layers "F.Cu" "B.Cu") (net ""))
 (via (at 3 15) (size 0.8) (drill 0.4) (layers "F.Cu" "B.Cu") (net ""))
 (via (at 27.5 2) (size 0.8) (drill 0.4) (layers "F.Cu" "B.Cu") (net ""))
 (via (at 27.5 13.5) (size 0.8) (drill 0.4) (layers "F.Cu" "B.Cu") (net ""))
 (via (at 11.5 17.5) (size 0.8) (drill 0.4) (layers "F.Cu" "B.Cu") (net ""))
 (via (at 28 20) (size 0.8) (drill 0.4) (layers "F.Cu" "B.Cu") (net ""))
 (via (at 20 16.5) (size 0.8) (drill 0.4) (layers "F.Cu" "B.Cu") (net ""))
 (via (at 25.5 8) (size 0.8) (drill 0.4) (layers "F.Cu" "B.Cu") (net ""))
 (via (at 16.5 25.5) (size 0.8) (drill 0.4) (layers "F.Cu" "B.Cu") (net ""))
 (via (at 24 19) (size 1) (drill 0.5) (layers "F.Cu" "B.Cu") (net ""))
 (via (at 13.5 16.5) (size 0.8) (drill 0.4) (layers "F.Cu" "B.Cu") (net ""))
 (via (at 13.25 23.7) (size 0.6) (drill 0.3) (layers "F.Cu" "B.Cu") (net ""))
 (via (at 1.5 5.46) (size 0.8) (drill 0.4) (layers "F.Cu" "B.Cu") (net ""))
 (via (at 14 25.5) (size 0.8) (drill 0.4) (layers "F.Cu" "B.Cu") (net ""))
 (via (at 18.6 17) (size 0.8) (drill 0.4) (layers "F.Cu" "B.Cu") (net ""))
 (via (at 14.5 26.5) (size 0.8) (drill 0.4) (layers "F.Cu" "B.Cu") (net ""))
 (via (at 8 15) (size 0.8) (drill 0.4) (layers "F.Cu" "B.Cu") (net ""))
 (segment (start 1.5 15.5) (end 13.5 15.5) (width 0.4) (layer "B.Cu") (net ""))
 (segment (start 13.5 15.5) (end 12 15.5) (width 0.4) (layer "B.Cu") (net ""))
 (segment (start 26.1 9.27) (end 26.1 20) (width 0.2) (layer "B.Cu") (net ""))
 (segment (start 26.8 4.19) (end 26.8 22) (width 0.2) (layer "B.Cu") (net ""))
 (segment (start 1.5 5.46) (end 1.5 15.5) (width 0.4) (layer "B.Cu") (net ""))
 (segment (start 25.1 8) (end 25.1 21) (width 0.2) (layer "B.Cu") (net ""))
 (segment (start 13.25 20) (end 13.25 23.7) (width 0.2) (layer "B.Cu") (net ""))
 (segment (start 12 15.5) (end 12 23) (width 0.4) (layer "B.Cu") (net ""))
 (segment (start 13.5 15.5) (end 18.6 15.5) (width 0.4) (layer "B.Cu") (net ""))
 (segment (start 24 19) (end 24 18.7) (width 1.5) (layer "B.Cu") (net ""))
 (segment (start 25.1 21) (end 14 21) (width 0.2) (layer "B.Cu") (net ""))
 (segment (start 26.8 22) (end 14.5 22) (width 0.2) (layer "B.Cu") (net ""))
 (segment (start 11.5 15.5) (end 11.5 17.5) (width 0.4) (layer "B.Cu") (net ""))
 (segment (start 18.6 15.5) (end 18.6 17) (width 0.4) (layer "B.Cu") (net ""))
 (segment (start 26.1 20) (end 13.25 20) (width 0.2) (layer "B.Cu") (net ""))
 (segment (start 14 21) (end 14 25.5) (width 0.2) (layer "B.Cu") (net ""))
 (segment (start 14.5 22) (end 14.5 26.5) (width 0.2) (layer "B.Cu") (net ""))
 (segment (start 25.5 8) (end 25.1 8) (width 0.2) (layer "B.Cu") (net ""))
 (segment (start 24 18.7) (end 3.5 18.7) (width 1.5) (layer "B.Cu") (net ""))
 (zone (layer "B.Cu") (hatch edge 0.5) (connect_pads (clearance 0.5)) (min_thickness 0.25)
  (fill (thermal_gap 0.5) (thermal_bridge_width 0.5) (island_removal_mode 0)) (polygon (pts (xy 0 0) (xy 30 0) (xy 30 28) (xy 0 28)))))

